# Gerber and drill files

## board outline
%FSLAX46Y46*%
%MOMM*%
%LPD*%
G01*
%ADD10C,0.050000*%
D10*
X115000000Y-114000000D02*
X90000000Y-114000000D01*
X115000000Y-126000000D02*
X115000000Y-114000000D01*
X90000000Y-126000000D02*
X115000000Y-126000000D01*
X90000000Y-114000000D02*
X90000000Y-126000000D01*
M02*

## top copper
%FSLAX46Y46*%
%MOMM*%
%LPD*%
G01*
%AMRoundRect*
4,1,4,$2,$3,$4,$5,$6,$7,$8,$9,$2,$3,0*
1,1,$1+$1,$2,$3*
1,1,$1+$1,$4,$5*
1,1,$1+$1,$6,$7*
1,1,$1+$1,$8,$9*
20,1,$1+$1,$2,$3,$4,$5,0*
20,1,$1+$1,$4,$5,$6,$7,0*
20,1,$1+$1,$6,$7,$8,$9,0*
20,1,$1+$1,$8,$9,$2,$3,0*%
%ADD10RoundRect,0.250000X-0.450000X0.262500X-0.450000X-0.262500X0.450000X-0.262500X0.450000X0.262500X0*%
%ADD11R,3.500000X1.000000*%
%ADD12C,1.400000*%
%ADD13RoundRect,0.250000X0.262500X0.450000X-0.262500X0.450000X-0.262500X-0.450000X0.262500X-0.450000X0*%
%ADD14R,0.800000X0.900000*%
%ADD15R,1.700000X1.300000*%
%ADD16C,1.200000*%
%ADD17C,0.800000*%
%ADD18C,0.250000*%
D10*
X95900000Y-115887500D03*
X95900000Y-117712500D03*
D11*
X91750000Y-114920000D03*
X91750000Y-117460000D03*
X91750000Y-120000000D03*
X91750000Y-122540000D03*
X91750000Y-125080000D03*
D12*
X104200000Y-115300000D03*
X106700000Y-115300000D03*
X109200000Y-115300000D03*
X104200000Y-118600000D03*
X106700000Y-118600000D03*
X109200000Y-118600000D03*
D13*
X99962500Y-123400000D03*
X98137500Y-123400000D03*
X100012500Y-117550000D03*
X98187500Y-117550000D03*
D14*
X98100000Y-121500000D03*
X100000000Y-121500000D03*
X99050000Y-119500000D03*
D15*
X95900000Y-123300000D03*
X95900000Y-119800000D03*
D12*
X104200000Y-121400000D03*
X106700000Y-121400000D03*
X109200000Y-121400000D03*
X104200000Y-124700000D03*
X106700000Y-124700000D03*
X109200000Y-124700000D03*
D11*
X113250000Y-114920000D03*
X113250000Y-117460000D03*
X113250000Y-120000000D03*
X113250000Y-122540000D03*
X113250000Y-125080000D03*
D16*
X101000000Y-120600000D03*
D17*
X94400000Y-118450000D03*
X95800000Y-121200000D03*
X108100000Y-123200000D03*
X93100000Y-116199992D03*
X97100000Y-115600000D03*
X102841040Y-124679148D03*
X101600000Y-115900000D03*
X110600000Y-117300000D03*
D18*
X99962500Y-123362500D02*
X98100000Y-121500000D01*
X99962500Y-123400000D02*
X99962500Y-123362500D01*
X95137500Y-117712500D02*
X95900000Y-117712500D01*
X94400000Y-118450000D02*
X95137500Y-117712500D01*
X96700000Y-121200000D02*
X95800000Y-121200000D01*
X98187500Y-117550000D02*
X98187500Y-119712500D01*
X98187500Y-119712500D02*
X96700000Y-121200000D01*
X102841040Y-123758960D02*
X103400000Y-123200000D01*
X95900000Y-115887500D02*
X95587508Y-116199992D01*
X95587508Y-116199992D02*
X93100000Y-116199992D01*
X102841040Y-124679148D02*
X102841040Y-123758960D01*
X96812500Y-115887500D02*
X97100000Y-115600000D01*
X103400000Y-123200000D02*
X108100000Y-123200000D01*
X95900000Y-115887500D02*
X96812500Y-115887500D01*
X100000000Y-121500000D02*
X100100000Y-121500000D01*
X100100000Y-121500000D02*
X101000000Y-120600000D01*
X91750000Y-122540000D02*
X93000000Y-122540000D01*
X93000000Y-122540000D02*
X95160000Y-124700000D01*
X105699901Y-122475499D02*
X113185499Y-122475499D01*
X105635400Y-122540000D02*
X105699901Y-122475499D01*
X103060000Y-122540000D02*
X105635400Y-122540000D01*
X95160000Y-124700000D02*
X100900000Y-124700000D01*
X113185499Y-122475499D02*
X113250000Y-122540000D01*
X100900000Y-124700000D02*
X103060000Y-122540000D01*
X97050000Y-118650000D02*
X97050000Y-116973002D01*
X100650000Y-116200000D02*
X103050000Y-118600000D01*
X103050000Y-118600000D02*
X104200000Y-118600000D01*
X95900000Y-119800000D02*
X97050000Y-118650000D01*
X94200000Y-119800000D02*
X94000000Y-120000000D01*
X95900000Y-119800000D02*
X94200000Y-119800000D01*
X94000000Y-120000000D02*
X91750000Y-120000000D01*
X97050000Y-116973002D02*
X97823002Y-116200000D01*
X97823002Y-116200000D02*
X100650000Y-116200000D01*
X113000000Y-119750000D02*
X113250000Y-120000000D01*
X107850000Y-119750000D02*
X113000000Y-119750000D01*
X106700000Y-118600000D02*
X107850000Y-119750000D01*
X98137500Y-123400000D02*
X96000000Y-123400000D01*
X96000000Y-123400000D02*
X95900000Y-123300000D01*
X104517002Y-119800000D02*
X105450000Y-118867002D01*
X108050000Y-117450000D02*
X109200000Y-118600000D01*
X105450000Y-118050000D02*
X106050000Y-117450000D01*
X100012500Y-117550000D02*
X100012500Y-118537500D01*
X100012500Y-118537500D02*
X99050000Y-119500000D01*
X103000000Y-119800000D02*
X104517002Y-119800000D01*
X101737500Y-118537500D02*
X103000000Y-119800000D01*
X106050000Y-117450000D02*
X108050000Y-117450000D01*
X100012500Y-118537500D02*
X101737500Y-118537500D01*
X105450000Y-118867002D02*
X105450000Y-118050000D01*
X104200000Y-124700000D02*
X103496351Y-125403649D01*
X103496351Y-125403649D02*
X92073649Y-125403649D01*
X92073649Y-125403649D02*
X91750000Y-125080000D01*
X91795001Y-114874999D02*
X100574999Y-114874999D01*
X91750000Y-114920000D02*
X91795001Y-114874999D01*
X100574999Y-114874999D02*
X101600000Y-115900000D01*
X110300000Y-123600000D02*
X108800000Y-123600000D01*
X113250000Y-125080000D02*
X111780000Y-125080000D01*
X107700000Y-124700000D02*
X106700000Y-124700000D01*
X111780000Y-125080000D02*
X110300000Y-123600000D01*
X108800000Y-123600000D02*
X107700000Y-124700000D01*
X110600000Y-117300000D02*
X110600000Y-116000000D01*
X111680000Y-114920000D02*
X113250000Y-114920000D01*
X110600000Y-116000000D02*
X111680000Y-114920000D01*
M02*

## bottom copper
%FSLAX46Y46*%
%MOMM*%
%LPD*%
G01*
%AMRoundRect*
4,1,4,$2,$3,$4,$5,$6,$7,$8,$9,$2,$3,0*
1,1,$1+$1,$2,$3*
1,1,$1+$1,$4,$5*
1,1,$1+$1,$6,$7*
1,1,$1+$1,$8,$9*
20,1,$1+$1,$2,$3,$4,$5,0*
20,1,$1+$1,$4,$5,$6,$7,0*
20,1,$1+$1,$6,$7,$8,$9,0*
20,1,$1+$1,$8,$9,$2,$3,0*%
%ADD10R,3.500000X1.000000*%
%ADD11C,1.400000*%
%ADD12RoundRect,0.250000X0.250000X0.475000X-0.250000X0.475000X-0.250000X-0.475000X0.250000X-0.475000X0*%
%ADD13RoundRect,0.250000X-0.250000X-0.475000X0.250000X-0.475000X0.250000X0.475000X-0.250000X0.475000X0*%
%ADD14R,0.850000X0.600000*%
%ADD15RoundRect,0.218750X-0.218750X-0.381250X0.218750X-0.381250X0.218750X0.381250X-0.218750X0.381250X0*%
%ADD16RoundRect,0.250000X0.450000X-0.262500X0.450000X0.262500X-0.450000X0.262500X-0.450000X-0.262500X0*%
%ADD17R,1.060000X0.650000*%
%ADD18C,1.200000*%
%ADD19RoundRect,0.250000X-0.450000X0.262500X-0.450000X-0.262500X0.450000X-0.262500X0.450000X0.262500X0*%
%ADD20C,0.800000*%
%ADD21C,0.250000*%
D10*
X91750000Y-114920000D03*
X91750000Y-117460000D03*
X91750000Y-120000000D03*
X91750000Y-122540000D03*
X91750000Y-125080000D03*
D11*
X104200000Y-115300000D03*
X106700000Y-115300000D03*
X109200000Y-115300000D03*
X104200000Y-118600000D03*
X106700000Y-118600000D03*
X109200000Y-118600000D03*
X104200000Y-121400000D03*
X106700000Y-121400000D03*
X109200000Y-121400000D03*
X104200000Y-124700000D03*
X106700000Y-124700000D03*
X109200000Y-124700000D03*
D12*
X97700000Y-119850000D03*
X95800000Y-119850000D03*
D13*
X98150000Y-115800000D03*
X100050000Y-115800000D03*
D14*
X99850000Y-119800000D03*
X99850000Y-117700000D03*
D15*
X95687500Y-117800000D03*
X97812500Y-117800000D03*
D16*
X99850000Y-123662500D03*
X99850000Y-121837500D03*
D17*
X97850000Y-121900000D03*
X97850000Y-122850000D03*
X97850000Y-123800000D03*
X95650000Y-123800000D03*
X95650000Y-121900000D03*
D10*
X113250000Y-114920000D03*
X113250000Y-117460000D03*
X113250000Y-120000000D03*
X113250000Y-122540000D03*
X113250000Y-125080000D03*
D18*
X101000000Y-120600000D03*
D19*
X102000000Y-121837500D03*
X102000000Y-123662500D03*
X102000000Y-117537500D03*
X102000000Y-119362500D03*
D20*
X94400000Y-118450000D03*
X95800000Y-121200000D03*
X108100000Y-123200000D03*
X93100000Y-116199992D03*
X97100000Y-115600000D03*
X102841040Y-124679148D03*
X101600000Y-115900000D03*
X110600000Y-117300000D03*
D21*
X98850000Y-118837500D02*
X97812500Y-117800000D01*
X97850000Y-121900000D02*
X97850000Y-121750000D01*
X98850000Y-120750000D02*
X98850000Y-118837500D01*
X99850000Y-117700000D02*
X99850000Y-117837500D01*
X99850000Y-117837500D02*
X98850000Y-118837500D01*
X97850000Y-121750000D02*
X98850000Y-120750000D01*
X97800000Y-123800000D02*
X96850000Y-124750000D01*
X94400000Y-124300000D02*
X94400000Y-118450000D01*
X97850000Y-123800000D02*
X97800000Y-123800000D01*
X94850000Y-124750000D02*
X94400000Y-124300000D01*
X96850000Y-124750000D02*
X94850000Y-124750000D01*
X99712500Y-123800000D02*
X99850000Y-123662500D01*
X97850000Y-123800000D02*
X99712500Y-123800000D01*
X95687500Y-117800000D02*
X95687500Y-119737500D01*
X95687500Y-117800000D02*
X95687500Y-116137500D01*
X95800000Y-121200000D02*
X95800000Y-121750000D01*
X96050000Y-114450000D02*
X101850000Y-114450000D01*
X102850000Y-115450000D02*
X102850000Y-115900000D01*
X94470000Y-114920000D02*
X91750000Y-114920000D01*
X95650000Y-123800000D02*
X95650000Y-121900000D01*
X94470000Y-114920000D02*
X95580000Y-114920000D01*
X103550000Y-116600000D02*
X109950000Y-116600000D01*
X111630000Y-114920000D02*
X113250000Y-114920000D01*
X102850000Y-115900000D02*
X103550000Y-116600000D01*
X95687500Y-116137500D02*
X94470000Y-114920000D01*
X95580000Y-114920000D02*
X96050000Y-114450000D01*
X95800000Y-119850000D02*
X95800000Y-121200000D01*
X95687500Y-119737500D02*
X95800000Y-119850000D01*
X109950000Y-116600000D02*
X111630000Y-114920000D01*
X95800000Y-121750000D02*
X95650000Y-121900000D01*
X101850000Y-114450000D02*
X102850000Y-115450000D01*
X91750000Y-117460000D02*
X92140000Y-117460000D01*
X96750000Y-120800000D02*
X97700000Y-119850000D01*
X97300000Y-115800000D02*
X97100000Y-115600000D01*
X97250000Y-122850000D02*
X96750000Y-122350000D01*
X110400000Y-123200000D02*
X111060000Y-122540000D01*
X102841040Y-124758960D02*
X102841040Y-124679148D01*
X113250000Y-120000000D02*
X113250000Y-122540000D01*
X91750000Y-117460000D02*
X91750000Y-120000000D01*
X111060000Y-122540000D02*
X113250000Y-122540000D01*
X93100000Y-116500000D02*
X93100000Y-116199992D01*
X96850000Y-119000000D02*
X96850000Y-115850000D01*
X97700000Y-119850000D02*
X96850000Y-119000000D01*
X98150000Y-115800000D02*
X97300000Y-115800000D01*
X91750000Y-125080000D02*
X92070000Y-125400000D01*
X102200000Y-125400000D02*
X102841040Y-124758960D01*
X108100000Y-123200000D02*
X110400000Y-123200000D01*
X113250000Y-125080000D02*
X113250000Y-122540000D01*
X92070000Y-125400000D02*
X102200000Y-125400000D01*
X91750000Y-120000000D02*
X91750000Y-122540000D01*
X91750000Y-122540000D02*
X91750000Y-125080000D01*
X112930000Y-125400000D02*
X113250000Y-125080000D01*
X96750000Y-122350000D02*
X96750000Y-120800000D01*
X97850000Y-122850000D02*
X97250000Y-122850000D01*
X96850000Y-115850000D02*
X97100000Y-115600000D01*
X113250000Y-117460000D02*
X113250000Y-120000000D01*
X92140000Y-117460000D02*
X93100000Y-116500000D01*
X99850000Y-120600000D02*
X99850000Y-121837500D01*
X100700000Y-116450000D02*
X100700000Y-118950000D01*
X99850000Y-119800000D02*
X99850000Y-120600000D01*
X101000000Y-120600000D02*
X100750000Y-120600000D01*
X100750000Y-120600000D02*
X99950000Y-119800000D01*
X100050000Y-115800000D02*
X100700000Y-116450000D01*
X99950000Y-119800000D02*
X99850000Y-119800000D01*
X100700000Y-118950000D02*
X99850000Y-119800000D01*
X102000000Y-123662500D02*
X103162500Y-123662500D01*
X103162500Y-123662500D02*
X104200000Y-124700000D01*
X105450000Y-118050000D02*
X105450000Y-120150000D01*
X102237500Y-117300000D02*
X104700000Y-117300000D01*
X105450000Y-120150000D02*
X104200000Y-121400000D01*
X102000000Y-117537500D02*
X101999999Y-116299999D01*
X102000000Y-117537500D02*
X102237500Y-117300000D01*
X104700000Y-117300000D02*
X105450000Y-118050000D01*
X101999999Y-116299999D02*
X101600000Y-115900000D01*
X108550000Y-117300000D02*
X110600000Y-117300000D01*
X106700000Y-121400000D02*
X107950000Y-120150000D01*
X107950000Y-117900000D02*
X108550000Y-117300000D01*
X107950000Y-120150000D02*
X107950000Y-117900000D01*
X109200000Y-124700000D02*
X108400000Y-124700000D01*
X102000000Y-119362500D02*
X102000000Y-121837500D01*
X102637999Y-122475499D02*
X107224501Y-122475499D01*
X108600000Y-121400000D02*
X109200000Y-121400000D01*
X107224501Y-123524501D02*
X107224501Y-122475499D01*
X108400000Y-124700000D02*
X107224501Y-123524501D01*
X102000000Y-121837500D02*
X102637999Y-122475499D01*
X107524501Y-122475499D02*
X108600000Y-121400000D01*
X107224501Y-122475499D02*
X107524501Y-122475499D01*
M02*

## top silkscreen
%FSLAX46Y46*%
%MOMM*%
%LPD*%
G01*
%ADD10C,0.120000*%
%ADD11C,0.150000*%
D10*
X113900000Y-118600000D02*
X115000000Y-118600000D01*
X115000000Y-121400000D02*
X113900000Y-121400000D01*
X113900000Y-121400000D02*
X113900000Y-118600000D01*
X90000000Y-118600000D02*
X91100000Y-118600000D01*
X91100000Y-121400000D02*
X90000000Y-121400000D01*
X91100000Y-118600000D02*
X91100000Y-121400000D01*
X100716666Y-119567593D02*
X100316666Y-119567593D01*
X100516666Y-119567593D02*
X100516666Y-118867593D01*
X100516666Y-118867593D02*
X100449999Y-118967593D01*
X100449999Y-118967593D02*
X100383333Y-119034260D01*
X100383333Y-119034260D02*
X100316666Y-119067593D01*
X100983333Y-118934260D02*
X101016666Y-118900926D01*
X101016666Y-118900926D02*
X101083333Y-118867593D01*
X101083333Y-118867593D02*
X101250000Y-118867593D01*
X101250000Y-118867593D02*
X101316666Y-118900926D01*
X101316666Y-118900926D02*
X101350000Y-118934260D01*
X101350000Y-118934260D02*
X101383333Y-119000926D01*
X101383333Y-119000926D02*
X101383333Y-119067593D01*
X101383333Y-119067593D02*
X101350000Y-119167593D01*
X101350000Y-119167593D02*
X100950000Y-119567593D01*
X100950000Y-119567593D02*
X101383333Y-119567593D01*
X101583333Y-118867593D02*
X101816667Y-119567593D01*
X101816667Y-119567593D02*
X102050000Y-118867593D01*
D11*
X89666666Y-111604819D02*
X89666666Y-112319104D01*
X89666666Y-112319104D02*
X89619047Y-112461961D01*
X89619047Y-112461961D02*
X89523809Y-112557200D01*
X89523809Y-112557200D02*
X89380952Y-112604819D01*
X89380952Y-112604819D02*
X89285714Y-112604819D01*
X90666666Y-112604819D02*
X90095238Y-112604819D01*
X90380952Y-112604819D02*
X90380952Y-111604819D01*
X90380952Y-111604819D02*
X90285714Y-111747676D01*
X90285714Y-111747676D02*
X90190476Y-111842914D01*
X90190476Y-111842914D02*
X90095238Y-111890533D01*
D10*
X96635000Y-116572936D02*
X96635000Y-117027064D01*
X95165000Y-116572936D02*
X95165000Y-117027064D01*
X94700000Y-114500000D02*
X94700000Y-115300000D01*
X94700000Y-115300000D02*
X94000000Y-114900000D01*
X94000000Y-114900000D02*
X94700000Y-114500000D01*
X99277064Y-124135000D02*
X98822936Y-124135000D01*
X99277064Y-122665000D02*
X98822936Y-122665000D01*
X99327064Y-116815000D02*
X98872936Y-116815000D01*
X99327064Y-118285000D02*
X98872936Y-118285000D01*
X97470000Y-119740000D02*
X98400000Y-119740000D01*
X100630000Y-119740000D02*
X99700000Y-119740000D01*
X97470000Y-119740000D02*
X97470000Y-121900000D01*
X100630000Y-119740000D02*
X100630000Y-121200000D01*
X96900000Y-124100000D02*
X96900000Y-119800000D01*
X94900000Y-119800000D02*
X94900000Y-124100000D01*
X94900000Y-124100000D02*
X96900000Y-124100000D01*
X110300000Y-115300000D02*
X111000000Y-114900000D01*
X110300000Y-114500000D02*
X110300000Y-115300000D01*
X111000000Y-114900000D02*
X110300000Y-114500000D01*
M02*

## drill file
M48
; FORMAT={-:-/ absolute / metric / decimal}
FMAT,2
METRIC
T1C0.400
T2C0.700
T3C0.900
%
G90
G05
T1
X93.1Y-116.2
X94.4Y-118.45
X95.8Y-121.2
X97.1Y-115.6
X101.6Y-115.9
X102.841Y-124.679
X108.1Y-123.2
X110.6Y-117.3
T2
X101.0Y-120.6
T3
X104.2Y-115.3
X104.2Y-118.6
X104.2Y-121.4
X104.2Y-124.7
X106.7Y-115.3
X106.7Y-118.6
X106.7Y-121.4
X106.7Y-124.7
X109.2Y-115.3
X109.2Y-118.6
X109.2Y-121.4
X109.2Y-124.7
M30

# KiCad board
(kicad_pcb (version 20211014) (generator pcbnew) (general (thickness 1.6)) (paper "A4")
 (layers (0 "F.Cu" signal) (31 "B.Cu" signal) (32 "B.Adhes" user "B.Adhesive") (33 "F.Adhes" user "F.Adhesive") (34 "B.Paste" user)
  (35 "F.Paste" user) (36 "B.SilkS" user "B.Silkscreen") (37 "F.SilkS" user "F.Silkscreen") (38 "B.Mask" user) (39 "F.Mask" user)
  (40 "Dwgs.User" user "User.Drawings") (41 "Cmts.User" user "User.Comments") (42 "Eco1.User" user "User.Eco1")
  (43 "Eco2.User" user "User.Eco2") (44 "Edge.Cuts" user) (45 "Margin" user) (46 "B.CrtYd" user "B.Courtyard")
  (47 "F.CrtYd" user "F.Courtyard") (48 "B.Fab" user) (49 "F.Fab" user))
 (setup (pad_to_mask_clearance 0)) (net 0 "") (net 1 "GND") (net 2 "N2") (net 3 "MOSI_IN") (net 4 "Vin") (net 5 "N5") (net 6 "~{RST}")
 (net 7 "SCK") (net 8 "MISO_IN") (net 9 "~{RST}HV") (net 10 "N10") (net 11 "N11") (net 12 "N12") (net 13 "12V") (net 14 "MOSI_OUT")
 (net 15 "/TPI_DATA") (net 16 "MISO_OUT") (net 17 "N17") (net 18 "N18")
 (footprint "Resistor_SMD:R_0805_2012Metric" (layer "F.Cu") (at 95.9 116.8 -90)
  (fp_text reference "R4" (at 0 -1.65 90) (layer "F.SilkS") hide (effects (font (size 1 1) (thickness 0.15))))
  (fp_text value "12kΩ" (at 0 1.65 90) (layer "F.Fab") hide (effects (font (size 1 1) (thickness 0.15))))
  (fp_line (start -0.227064 -0.735) (end 0.227064 -0.735) (layer "F.SilkS") (width 0.12))
  (fp_line (start -0.227064 0.735) (end 0.227064 0.735) (layer "F.SilkS") (width 0.12))
  (pad "1" smd roundrect locked (at -0.9125 0 270) (size 1.025 1.4) (layers "F.Cu" "F.Paste" "F.Mask") (roundrect_rratio 0.243902)
   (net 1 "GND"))
  (pad "2" smd roundrect locked (at 0.9125 0 270) (size 1.025 1.4) (layers "F.Cu" "F.Paste" "F.Mask") (roundrect_rratio 0.243902)
   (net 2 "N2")))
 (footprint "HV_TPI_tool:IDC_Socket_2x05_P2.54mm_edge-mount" (layer "F.Cu") (at 90 120)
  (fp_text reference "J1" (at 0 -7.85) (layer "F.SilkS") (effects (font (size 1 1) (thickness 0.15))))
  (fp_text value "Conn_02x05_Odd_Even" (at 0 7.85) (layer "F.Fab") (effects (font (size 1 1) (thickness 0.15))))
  (fp_line (start 4.7 -5.5) (end 4.7 -4.7) (layer "F.SilkS") (width 0.12))
  (fp_line (start 4.7 -4.7) (end 4 -5.1) (layer "F.SilkS") (width 0.12))
  (fp_line (start 4 -5.1) (end 4.7 -5.5) (layer "F.SilkS") (width 0.12))
  (pad "1" smd rect (at 1.75 -5.08) (size 3.5 1) (layers "F.Cu" "F.Paste" "F.Mask") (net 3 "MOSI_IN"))
  (pad "2" smd rect (at 1.75 -5.08) (size 3.5 1) (layers "B.Cu" "B.Paste" "B.Mask") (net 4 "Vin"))
  (pad "3" smd rect (at 1.75 -2.54) (size 3.5 1) (layers "F.Cu" "F.Paste" "F.Mask") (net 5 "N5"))
  (pad "4" smd rect (at 1.75 -2.54) (size 3.5 1) (layers "B.Cu" "B.Paste" "B.Mask") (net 1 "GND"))
  (pad "5" smd rect (at 1.75 0) (size 3.5 1) (layers "F.Cu" "F.Paste" "F.Mask") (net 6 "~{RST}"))
  (pad "6" smd rect (at 1.75 0) (size 3.5 1) (layers "B.Cu" "B.Paste" "B.Mask") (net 1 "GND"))
  (pad "7" smd rect (at 1.75 2.54) (size 3.5 1) (layers "F.Cu" "F.Paste" "F.Mask") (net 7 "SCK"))
  (pad "8" smd rect (at 1.75 2.54) (size 3.5 1) (layers "B.Cu" "B.Paste" "B.Mask") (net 1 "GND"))
  (pad "9" smd rect (at 1.75 5.08) (size 3.5 1) (layers "F.Cu" "F.Paste" "F.Mask") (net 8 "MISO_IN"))
  (pad "10" smd rect (at 1.75 5.08) (size 3.5 1) (layers "B.Cu" "B.Paste" "B.Mask") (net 1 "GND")))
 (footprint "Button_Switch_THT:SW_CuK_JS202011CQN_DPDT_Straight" (layer "F.Cu") (at 104.2 115.3)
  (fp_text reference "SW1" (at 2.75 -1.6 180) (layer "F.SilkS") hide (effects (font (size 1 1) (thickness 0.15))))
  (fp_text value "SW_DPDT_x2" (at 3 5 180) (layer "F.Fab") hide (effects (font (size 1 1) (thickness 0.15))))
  (pad "1" thru_hole circle locked (at 0 0) (size 1.4 1.4) (drill 0.9) (layers *.Cu *.Mask))
  (pad "2" thru_hole circle locked (at 2.5 0) (size 1.4 1.4) (drill 0.9) (layers *.Cu *.Mask))
  (pad "3" thru_hole circle locked (at 5 0) (size 1.4 1.4) (drill 0.9) (layers *.Cu *.Mask))
  (pad "4" thru_hole circle locked (at 0 3.3) (size 1.4 1.4) (drill 0.9) (layers *.Cu *.Mask) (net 6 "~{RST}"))
  (pad "5" thru_hole circle locked (at 2.5 3.3) (size 1.4 1.4) (drill 0.9) (layers *.Cu *.Mask) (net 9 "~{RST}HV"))
  (pad "6" thru_hole circle locked (at 5 3.3) (size 1.4 1.4) (drill 0.9) (layers *.Cu *.Mask) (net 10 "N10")))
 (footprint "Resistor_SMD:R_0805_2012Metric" (layer "F.Cu") (at 99.05 123.4 180)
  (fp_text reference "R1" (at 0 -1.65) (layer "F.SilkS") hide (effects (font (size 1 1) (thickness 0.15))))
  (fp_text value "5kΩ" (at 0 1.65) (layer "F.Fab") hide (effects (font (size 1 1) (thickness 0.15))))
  (fp_line (start -0.227064 -0.735) (end 0.227064 -0.735) (layer "F.SilkS") (width 0.12))
  (fp_line (start -0.227064 0.735) (end 0.227064 0.735) (layer "F.SilkS") (width 0.12))
  (pad "1" smd roundrect locked (at -0.9125 0 180) (size 1.025 1.4) (layers "F.Cu" "F.Paste" "F.Mask") (roundrect_rratio 0.243902)
   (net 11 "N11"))
  (pad "2" smd roundrect locked (at 0.9125 0 180) (size 1.025 1.4) (layers "F.Cu" "F.Paste" "F.Mask") (roundrect_rratio 0.243902)
   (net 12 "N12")))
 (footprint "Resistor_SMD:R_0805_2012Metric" (layer "F.Cu") (at 99.1 117.55 180)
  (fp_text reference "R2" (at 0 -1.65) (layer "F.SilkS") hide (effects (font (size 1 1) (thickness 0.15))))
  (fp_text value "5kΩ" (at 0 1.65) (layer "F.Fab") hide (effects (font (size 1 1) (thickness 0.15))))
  (fp_line (start -0.227064 0.735) (end 0.227064 0.735) (layer "F.SilkS") (width 0.12))
  (fp_line (start -0.227064 -0.735) (end 0.227064 -0.735) (layer "F.SilkS") (width 0.12))
  (pad "1" smd roundrect locked (at -0.9125 0 180) (size 1.025 1.4) (layers "F.Cu" "F.Paste" "F.Mask") (roundrect_rratio 0.243902)
   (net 10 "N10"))
  (pad "2" smd roundrect locked (at 0.9125 0 180) (size 1.025 1.4) (layers "F.Cu" "F.Paste" "F.Mask") (roundrect_rratio 0.243902)
   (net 4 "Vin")))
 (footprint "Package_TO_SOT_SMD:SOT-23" (layer "F.Cu") (at 99.05 120.5 90)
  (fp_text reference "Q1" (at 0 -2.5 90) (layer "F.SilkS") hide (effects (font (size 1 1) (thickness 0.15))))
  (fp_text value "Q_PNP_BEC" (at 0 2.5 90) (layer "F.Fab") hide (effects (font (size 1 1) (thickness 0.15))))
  (fp_line (start 0.76 -1.58) (end 0.76 -0.65) (layer "F.SilkS") (width 0.12))
  (fp_line (start 0.76 1.58) (end 0.76 0.65) (layer "F.SilkS") (width 0.12))
  (fp_line (start 0.76 -1.58) (end -1.4 -1.58) (layer "F.SilkS") (width 0.12))
  (fp_line (start 0.76 1.58) (end -0.7 1.58) (layer "F.SilkS") (width 0.12))
  (pad "1" smd rect locked (at -1 -0.95 90) (size 0.9 0.8) (layers "F.Cu" "F.Paste" "F.Mask") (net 11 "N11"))
  (pad "2" smd rect locked (at -1 0.95 90) (size 0.9 0.8) (layers "F.Cu" "F.Paste" "F.Mask") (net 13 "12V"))
  (pad "3" smd rect locked (at 1 0 90) (size 0.9 0.8) (layers "F.Cu" "F.Paste" "F.Mask") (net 10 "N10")))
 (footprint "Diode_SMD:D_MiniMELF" (layer "F.Cu") (at 95.9 121.55 90)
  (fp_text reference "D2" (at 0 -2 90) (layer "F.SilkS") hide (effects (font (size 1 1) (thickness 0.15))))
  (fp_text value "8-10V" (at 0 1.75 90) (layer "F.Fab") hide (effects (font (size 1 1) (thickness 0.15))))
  (fp_line (start -2.55 1) (end 1.75 1) (layer "F.SilkS") (width 0.12))
  (fp_line (start 1.75 -1) (end -2.55 -1) (layer "F.SilkS") (width 0.12))
  (fp_line (start -2.55 -1) (end -2.55 1) (layer "F.SilkS") (width 0.12))
  (pad "1" smd rect locked (at -1.75 0 90) (size 1.3 1.7) (layers "F.Cu" "F.Paste" "F.Mask") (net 12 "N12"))
  (pad "2" smd rect locked (at 1.75 0 90) (size 1.3 1.7) (layers "F.Cu" "F.Paste" "F.Mask") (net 6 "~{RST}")))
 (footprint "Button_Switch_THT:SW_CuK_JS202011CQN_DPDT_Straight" (layer "F.Cu") (at 104.2 121.4)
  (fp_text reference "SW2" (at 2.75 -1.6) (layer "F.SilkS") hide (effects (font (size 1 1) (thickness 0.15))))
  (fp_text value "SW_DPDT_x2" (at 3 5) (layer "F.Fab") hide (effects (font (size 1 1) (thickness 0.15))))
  (pad "1" thru_hole circle (at 0 0) (size 1.4 1.4) (drill 0.9) (layers *.Cu *.Mask) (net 3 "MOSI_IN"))
  (pad "2" thru_hole circle (at 2.5 0) (size 1.4 1.4) (drill 0.9) (layers *.Cu *.Mask) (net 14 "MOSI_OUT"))
  (pad "3" thru_hole circle (at 5 0) (size 1.4 1.4) (drill 0.9) (layers *.Cu *.Mask) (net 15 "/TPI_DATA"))
  (pad "4" thru_hole circle (at 0 3.3) (size 1.4 1.4) (drill 0.9) (layers *.Cu *.Mask) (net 8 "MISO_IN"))
  (pad "5" thru_hole circle (at 2.5 3.3) (size 1.4 1.4) (drill 0.9) (layers *.Cu *.Mask) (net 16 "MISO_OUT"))
  (pad "6" thru_hole circle (at 5 3.3) (size 1.4 1.4) (drill 0.9) (layers *.Cu *.Mask) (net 15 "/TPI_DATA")))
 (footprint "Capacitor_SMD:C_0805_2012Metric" (layer "B.Cu") (at 96.75 119.85 180)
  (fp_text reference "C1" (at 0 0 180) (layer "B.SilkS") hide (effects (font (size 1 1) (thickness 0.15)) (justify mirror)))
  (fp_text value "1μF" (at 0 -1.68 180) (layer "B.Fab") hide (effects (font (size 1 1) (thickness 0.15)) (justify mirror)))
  (pad "1" smd roundrect locked (at -0.95 0 180) (size 1 1.45) (layers "B.Cu" "B.Paste" "B.Mask") (roundrect_rratio 0.25) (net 1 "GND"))
  (pad "2" smd roundrect locked (at 0.95 0 180) (size 1 1.45) (layers "B.Cu" "B.Paste" "B.Mask") (roundrect_rratio 0.25) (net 4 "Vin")))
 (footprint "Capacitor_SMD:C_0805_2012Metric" (layer "B.Cu") (at 99.1 115.8)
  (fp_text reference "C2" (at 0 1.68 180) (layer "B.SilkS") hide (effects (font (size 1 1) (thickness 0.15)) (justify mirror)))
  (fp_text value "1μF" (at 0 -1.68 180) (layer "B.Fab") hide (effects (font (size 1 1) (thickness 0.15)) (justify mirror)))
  (pad "1" smd roundrect locked (at -0.95 0) (size 1 1.45) (layers "B.Cu" "B.Paste" "B.Mask") (roundrect_rratio 0.25) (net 1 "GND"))
  (pad "2" smd roundrect locked (at 0.95 0) (size 1 1.45) (layers "B.Cu" "B.Paste" "B.Mask") (roundrect_rratio 0.25) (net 13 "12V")))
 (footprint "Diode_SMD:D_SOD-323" (layer "B.Cu") (at 99.85 118.75 90)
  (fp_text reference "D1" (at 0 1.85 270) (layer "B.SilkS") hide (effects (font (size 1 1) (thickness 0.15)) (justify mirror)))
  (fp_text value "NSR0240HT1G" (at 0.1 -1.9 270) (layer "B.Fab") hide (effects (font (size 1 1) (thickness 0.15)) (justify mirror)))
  (pad "1" smd rect locked (at -1.05 0 90) (size 0.6 0.85) (layers "B.Cu" "B.Paste" "B.Mask") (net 13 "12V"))
  (pad "2" smd rect locked (at 1.05 0 90) (size 0.6 0.85) (layers "B.Cu" "B.Paste" "B.Mask") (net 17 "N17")))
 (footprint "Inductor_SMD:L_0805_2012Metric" (layer "B.Cu") (at 96.75 117.8)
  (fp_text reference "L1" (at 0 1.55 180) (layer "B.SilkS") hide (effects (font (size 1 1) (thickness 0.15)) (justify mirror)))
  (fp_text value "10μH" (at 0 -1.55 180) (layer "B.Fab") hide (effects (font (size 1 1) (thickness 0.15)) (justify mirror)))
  (pad "1" smd roundrect locked (at -1.0625 0) (size 0.875 1.2) (layers "B.Cu" "B.Paste" "B.Mask") (roundrect_rratio 0.25) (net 4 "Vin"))
  (pad "2" smd roundrect locked (at 1.0625 0) (size 0.875 1.2) (layers "B.Cu" "B.Paste" "B.Mask") (roundrect_rratio 0.25) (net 17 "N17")))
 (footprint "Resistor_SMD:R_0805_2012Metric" (layer "B.Cu") (at 99.85 122.75 90)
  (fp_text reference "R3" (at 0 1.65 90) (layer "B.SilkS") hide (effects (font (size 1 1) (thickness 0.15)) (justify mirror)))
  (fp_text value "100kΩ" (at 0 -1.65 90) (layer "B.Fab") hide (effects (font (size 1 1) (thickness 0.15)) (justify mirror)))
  (pad "1" smd roundrect locked (at -0.9125 0 90) (size 1.025 1.4) (layers "B.Cu" "B.Paste" "B.Mask") (roundrect_rratio 0.243902)
   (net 2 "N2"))
  (pad "2" smd roundrect locked (at 0.9125 0 90) (size 1.025 1.4) (layers "B.Cu" "B.Paste" "B.Mask") (roundrect_rratio 0.243902)
   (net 13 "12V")))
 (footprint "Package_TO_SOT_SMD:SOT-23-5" (layer "B.Cu") (at 96.75 122.85 180)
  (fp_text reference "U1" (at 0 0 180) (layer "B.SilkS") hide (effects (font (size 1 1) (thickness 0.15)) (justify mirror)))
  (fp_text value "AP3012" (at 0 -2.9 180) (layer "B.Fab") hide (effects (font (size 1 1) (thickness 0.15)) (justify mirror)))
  (pad "1" smd rect locked (at -1.1 0.95 180) (size 1.06 0.65) (layers "B.Cu" "B.Paste" "B.Mask") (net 17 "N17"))
  (pad "2" smd rect locked (at -1.1 0 180) (size 1.06 0.65) (layers "B.Cu" "B.Paste" "B.Mask") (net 1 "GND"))
  (pad "3" smd rect locked (at -1.1 -0.95 180) (size 1.06 0.65) (layers "B.Cu" "B.Paste" "B.Mask") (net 2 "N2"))
  (pad "4" smd rect locked (at 1.1 -0.95 180) (size 1.06 0.65) (layers "B.Cu" "B.Paste" "B.Mask") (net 4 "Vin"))
  (pad "5" smd rect locked (at 1.1 0.95 180) (size 1.06 0.65) (layers "B.Cu" "B.Paste" "B.Mask") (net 4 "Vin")))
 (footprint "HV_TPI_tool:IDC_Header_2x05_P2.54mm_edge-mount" (layer "B.Cu") (at 115 120 180)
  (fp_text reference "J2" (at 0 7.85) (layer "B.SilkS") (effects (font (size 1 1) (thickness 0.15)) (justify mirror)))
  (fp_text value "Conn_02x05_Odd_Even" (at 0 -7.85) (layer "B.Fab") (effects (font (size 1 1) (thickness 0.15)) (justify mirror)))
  (fp_line (start 4.7 4.7) (end 4 5.1) (layer "F.SilkS") (width 0.12))
  (fp_line (start 4.7 5.5) (end 4.7 4.7) (layer "F.SilkS") (width 0.12))
  (fp_line (start 4 5.1) (end 4.7 5.5) (layer "F.SilkS") (width 0.12))
  (pad "1" smd rect (at 1.75 5.08 180) (size 3.5 1) (layers "F.Cu" "F.Paste" "F.Mask") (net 14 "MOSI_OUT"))
  (pad "2" smd rect (at 1.75 5.08 180) (size 3.5 1) (layers "B.Cu" "B.Paste" "B.Mask") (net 4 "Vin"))
  (pad "3" smd rect (at 1.75 2.54 180) (size 3.5 1) (layers "F.Cu" "F.Paste" "F.Mask") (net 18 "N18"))
  (pad "4" smd rect (at 1.75 2.54 180) (size 3.5 1) (layers "B.Cu" "B.Paste" "B.Mask") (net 1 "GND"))
  (pad "5" smd rect (at 1.75 0 180) (size 3.5 1) (layers "F.Cu" "F.Paste" "F.Mask") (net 9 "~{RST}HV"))
  (pad "6" smd rect (at 1.75 0 180) (size 3.5 1) (layers "B.Cu" "B.Paste" "B.Mask") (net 1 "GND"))
  (pad "7" smd rect (at 1.75 -2.54 180) (size 3.5 1) (layers "F.Cu" "F.Paste" "F.Mask") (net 7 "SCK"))
  (pad "8" smd rect (at 1.75 -2.54 180) (size 3.5 1) (layers "B.Cu" "B.Paste" "B.Mask") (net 1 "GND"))
  (pad "9" smd rect (at 1.75 -5.08 180) (size 3.5 1) (layers "F.Cu" "F.Paste" "F.Mask") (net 16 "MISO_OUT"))
  (pad "10" smd rect (at 1.75 -5.08 180) (size 3.5 1) (layers "B.Cu" "B.Paste" "B.Mask") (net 1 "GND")))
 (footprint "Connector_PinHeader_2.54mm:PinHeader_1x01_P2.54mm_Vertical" (layer "B.Cu") (at 101 120.6)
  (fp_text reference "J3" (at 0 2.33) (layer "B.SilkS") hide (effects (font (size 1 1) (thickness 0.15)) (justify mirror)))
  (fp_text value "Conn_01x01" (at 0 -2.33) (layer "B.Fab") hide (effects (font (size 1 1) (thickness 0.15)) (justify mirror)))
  (pad "1" thru_hole circle locked (at 0 0) (size 1.2 1.2) (drill 0.7) (layers *.Cu *.Mask) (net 13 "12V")))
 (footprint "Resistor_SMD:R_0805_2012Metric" (layer "B.Cu") (at 102 122.75 -90)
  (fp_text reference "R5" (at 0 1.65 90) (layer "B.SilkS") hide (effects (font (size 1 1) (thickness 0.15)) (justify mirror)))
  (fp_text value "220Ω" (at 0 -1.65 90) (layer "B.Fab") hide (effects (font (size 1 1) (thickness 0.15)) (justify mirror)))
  (pad "1" smd roundrect locked (at -0.9125 0 270) (size 1.025 1.4) (layers "B.Cu" "B.Paste" "B.Mask") (roundrect_rratio 0.243902)
   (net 15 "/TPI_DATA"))
  (pad "2" smd roundrect locked (at 0.9125 0 270) (size 1.025 1.4) (layers "B.Cu" "B.Paste" "B.Mask") (roundrect_rratio 0.243902)
   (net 8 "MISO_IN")))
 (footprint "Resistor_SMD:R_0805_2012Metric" (layer "B.Cu") (at 102 118.45 -90)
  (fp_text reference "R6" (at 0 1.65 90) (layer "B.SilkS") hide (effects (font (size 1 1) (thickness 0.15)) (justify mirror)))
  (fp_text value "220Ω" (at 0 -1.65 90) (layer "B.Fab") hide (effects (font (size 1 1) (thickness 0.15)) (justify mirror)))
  (pad "1" smd roundrect locked (at -0.9125 0 270) (size 1.025 1.4) (layers "B.Cu" "B.Paste" "B.Mask") (roundrect_rratio 0.243902)
   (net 3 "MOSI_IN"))
  (pad "2" smd roundrect locked (at 0.9125 0 270) (size 1.025 1.4) (layers "B.Cu" "B.Paste" "B.Mask") (roundrect_rratio 0.243902)
   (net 15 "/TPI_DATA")))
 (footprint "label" (layer "B.Cu") (at 94.35 119.95 -90)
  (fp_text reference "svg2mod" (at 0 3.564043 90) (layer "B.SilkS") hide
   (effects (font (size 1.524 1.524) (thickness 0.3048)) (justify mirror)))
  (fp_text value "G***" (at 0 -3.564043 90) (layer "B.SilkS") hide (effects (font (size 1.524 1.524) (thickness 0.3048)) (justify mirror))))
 (gr_line (start 113.9 118.6) (end 115 118.6) (layer "F.SilkS") (width 0.12))
 (gr_line (start 115 121.4) (end 113.9 121.4) (layer "F.SilkS") (width 0.12))
 (gr_line (start 113.9 121.4) (end 113.9 118.6) (layer "F.SilkS") (width 0.12))
 (gr_line (start 90 118.6) (end 91.1 118.6) (layer "F.SilkS") (width 0.12))
 (gr_line (start 91.1 121.4) (end 90 121.4) (layer "F.SilkS") (width 0.12))
 (gr_line (start 91.1 118.6) (end 91.1 121.4) (layer "F.SilkS") (width 0.12))
 (gr_line (start 115 114) (end 90 114) (layer "Edge.Cuts") (width 0.05))
 (gr_line (start 115 126) (end 115 114) (layer "Edge.Cuts") (width 0.05))
 (gr_line (start 90 126) (end 115 126) (layer "Edge.Cuts") (width 0.05))
 (gr_line (start 90 114) (end 90 126) (layer "Edge.Cuts") (width 0.05))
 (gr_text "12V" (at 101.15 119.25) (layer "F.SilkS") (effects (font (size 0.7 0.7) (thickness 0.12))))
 (segment (start 99.9625 123.3625) (end 98.1 121.5) (width 0.25) (layer "F.Cu") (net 11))
 (segment (start 99.9625 123.4) (end 99.9625 123.3625) (width 0.25) (layer "F.Cu") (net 11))
 (segment (start 98.85 118.8375) (end 97.8125 117.8) (width 0.25) (layer "B.Cu") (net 17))
 (segment (start 97.85 121.9) (end 97.85 121.75) (width 0.25) (layer "B.Cu") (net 17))
 (segment (start 98.85 120.75) (end 98.85 118.8375) (width 0.25) (layer "B.Cu") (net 17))
 (segment (start 99.85 117.7) (end 99.85 117.8375) (width 0.25) (layer "B.Cu") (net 17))
 (segment (start 99.85 117.8375) (end 98.85 118.8375) (width 0.25) (layer "B.Cu") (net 17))
 (segment (start 97.85 121.75) (end 98.85 120.75) (width 0.25) (layer "B.Cu") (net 17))
 (segment (start 95.1375 117.7125) (end 95.9 117.7125) (width 0.25) (layer "F.Cu") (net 2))
 (segment (start 94.4 118.45) (end 95.1375 117.7125) (width 0.25) (layer "F.Cu") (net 2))
 (via (at 94.4 118.45) (size 0.8) (drill 0.4) (layers "F.Cu" "B.Cu") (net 2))
 (segment (start 97.8 123.8) (end 96.85 124.75) (width 0.25) (layer "B.Cu") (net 2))
 (segment (start 94.4 124.3) (end 94.4 118.45) (width 0.25) (layer "B.Cu") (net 2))
 (segment (start 97.85 123.8) (end 97.8 123.8) (width 0.25) (layer "B.Cu") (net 2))
 (segment (start 94.85 124.75) (end 94.4 124.3) (width 0.25) (layer "B.Cu") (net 2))
 (segment (start 96.85 124.75) (end 94.85 124.75) (width 0.25) (layer "B.Cu") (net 2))
 (segment (start 99.7125 123.8) (end 99.85 123.6625) (width 0.25) (layer "B.Cu") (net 2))
 (segment (start 97.85 123.8) (end 99.7125 123.8) (width 0.25) (layer "B.Cu") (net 2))
 (segment (start 96.7 121.2) (end 95.8 121.2) (width 0.25) (layer "F.Cu") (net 4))
 (segment (start 98.1875 117.55) (end 98.1875 119.7125) (width 0.25) (layer "F.Cu") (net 4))
 (segment (start 98.1875 119.7125) (end 96.7 121.2) (width 0.25) (layer "F.Cu") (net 4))
 (via (at 95.8 121.2) (size 0.8) (drill 0.4) (layers "F.Cu" "B.Cu") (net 4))
 (segment (start 95.6875 117.8) (end 95.6875 119.7375) (width 0.25) (layer "B.Cu") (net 4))
 (segment (start 95.6875 117.8) (end 95.6875 116.1375) (width 0.25) (layer "B.Cu") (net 4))
 (segment (start 95.8 121.2) (end 95.8 121.75) (width 0.25) (layer "B.Cu") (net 4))
 (segment (start 96.05 114.45) (end 101.85 114.45) (width 0.25) (layer "B.Cu") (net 4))
 (segment (start 102.85 115.45) (end 102.85 115.9) (width 0.25) (layer "B.Cu") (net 4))
 (segment (start 94.47 114.92) (end 91.75 114.92) (width 0.25) (layer "B.Cu") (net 4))
 (segment (start 95.65 123.8) (end 95.65 121.9) (width 0.25) (layer "B.Cu") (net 4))
 (segment (start 94.47 114.92) (end 95.58 114.92) (width 0.25) (layer "B.Cu") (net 4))
 (segment (start 103.55 116.6) (end 109.95 116.6) (width 0.25) (layer "B.Cu") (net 4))
 (segment (start 111.63 114.92) (end 113.25 114.92) (width 0.25) (layer "B.Cu") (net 4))
 (segment (start 102.85 115.9) (end 103.55 116.6) (width 0.25) (layer "B.Cu") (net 4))
 (segment (start 95.6875 116.1375) (end 94.47 114.92) (width 0.25) (layer "B.Cu") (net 4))
 (segment (start 95.58 114.92) (end 96.05 114.45) (width 0.25) (layer "B.Cu") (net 4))
 (segment (start 95.8 119.85) (end 95.8 121.2) (width 0.25) (layer "B.Cu") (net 4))
 (segment (start 95.6875 119.7375) (end 95.8 119.85) (width 0.25) (layer "B.Cu") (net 4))
 (segment (start 109.95 116.6) (end 111.63 114.92) (width 0.25) (layer "B.Cu") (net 4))
 (segment (start 95.8 121.75) (end 95.65 121.9) (width 0.25) (layer "B.Cu") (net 4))
 (segment (start 101.85 114.45) (end 102.85 115.45) (width 0.25) (layer "B.Cu") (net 4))
 (segment (start 102.84104 123.75896) (end 103.4 123.2) (width 0.25) (layer "F.Cu") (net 1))
 (segment (start 95.9 115.8875) (end 95.587508 116.199992) (width 0.25) (layer "F.Cu") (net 1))
 (segment (start 95.587508 116.199992) (end 93.1 116.199992) (width 0.25) (layer "F.Cu") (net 1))
 (segment (start 102.84104 124.679148) (end 102.84104 123.75896) (width 0.25) (layer "F.Cu") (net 1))
 (segment (start 96.8125 115.8875) (end 97.1 115.6) (width 0.25) (layer "F.Cu") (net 1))
 (segment (start 103.4 123.2) (end 108.1 123.2) (width 0.25) (layer "F.Cu") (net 1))
 (segment (start 95.9 115.8875) (end 96.8125 115.8875) (width 0.25) (layer "F.Cu") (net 1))
 (via (at 108.1 123.2) (size 0.8) (drill 0.4) (layers "F.Cu" "B.Cu") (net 1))
 (via (at 93.1 116.199992) (size 0.8) (drill 0.4) (layers "F.Cu" "B.Cu") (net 1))
 (via (at 97.1 115.6) (size 0.8) (drill 0.4) (layers "F.Cu" "B.Cu") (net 1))
 (via (at 102.84104 124.679148) (size 0.8) (drill 0.4) (layers "F.Cu" "B.Cu") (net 1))
 (segment (start 91.75 117.46) (end 92.14 117.46) (width 0.25) (layer "B.Cu") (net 1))
 (segment (start 96.75 120.8) (end 97.7 119.85) (width 0.25) (layer "B.Cu") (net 1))
 (segment (start 97.3 115.8) (end 97.1 115.6) (width 0.25) (layer "B.Cu") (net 1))
 (segment (start 97.25 122.85) (end 96.75 122.35) (width 0.25) (layer "B.Cu") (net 1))
 (segment (start 110.4 123.2) (end 111.06 122.54) (width 0.25) (layer "B.Cu") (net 1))
 (segment (start 102.84104 124.75896) (end 102.84104 124.679148) (width 0.25) (layer "B.Cu") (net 1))
 (segment (start 113.25 120) (end 113.25 122.54) (width 0.25) (layer "B.Cu") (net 1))
 (segment (start 91.75 117.46) (end 91.75 120) (width 0.25) (layer "B.Cu") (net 1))
 (segment (start 111.06 122.54) (end 113.25 122.54) (width 0.25) (layer "B.Cu") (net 1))
 (segment (start 93.1 116.5) (end 93.1 116.199992) (width 0.25) (layer "B.Cu") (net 1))
 (segment (start 96.85 119) (end 96.85 115.85) (width 0.25) (layer "B.Cu") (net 1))
 (segment (start 97.7 119.85) (end 96.85 119) (width 0.25) (layer "B.Cu") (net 1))
 (segment (start 98.15 115.8) (end 97.3 115.8) (width 0.25) (layer "B.Cu") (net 1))
 (segment (start 91.75 125.08) (end 92.07 125.4) (width 0.25) (layer "B.Cu") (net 1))
 (segment (start 102.2 125.4) (end 102.84104 124.75896) (width 0.25) (layer "B.Cu") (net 1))
 (segment (start 108.1 123.2) (end 110.4 123.2) (width 0.25) (layer "B.Cu") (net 1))
 (segment (start 113.25 125.08) (end 113.25 122.54) (width 0.25) (layer "B.Cu") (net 1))
 (segment (start 92.07 125.4) (end 102.2 125.4) (width 0.25) (layer "B.Cu") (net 1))
 (segment (start 91.75 120) (end 91.75 122.54) (width 0.25) (layer "B.Cu") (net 1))
 (segment (start 91.75 122.54) (end 91.75 125.08) (width 0.25) (layer "B.Cu") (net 1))
 (segment (start 112.93 125.4) (end 113.25 125.08) (width 0.25) (layer "B.Cu") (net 1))
 (segment (start 96.75 122.35) (end 96.75 120.8) (width 0.25) (layer "B.Cu") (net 1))
 (segment (start 97.85 122.85) (end 97.25 122.85) (width 0.25) (layer "B.Cu") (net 1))
 (segment (start 96.85 115.85) (end 97.1 115.6) (width 0.25) (layer "B.Cu") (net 1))
 (segment (start 113.25 117.46) (end 113.25 120) (width 0.25) (layer "B.Cu") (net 1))
 (segment (start 92.14 117.46) (end 93.1 116.5) (width 0.25) (layer "B.Cu") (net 1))
 (segment (start 100 121.5) (end 100.1 121.5) (width 0.25) (layer "F.Cu") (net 13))
 (segment (start 100.1 121.5) (end 101 120.6) (width 0.25) (layer "F.Cu") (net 13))
 (segment (start 99.85 120.6) (end 99.85 121.8375) (width 0.25) (layer "B.Cu") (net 13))
 (segment (start 100.7 116.45) (end 100.7 118.95) (width 0.25) (layer "B.Cu") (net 13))
 (segment (start 99.85 119.8) (end 99.85 120.6) (width 0.25) (layer "B.Cu") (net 13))
 (segment (start 101 120.6) (end 100.75 120.6) (width 0.25) (layer "B.Cu") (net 13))
 (segment (start 100.75 120.6) (end 99.95 119.8) (width 0.25) (layer "B.Cu") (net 13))
 (segment (start 100.05 115.8) (end 100.7 116.45) (width 0.25) (layer "B.Cu") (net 13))
 (segment (start 99.95 119.8) (end 99.85 119.8) (width 0.25) (layer "B.Cu") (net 13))
 (segment (start 100.7 118.95) (end 99.85 119.8) (width 0.25) (layer "B.Cu") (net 13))
 (segment (start 91.75 122.54) (end 93 122.54) (width 0.25) (layer "F.Cu") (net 7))
 (segment (start 93 122.54) (end 95.16 124.7) (width 0.25) (layer "F.Cu") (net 7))
 (segment (start 105.699901 122.475499) (end 113.185499 122.475499) (width 0.25) (layer "F.Cu") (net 7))
 (segment (start 105.6354 122.54) (end 105.699901 122.475499) (width 0.25) (layer "F.Cu") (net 7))
 (segment (start 103.06 122.54) (end 105.6354 122.54) (width 0.25) (layer "F.Cu") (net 7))
 (segment (start 95.16 124.7) (end 100.9 124.7) (width 0.25) (layer "F.Cu") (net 7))
 (segment (start 113.185499 122.475499) (end 113.25 122.54) (width 0.25) (layer "F.Cu") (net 7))
 (segment (start 100.9 124.7) (end 103.06 122.54) (width 0.25) (layer "F.Cu") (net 7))
 (segment (start 97.05 118.65) (end 97.05 116.973002) (width 0.25) (layer "F.Cu") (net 6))
 (segment (start 100.65 116.2) (end 103.05 118.6) (width 0.25) (layer "F.Cu") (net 6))
 (segment (start 103.05 118.6) (end 104.2 118.6) (width 0.25) (layer "F.Cu") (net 6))
 (segment (start 95.9 119.8) (end 97.05 118.65) (width 0.25) (layer "F.Cu") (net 6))
 (segment (start 94.2 119.8) (end 94 120) (width 0.25) (layer "F.Cu") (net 6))
 (segment (start 95.9 119.8) (end 94.2 119.8) (width 0.25) (layer "F.Cu") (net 6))
 (segment (start 94 120) (end 91.75 120) (width 0.25) (layer "F.Cu") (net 6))
 (segment (start 97.05 116.973002) (end 97.823002 116.2) (width 0.25) (layer "F.Cu") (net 6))
 (segment (start 97.823002 116.2) (end 100.65 116.2) (width 0.25) (layer "F.Cu") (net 6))
 (segment (start 113 119.75) (end 113.25 120) (width 0.25) (layer "F.Cu") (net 9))
 (segment (start 107.85 119.75) (end 113 119.75) (width 0.25) (layer "F.Cu") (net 9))
 (segment (start 106.7 118.6) (end 107.85 119.75) (width 0.25) (layer "F.Cu") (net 9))
 (segment (start 98.1375 123.4) (end 96 123.4) (width 0.25) (layer "F.Cu") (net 12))
 (segment (start 96 123.4) (end 95.9 123.3) (width 0.25) (layer "F.Cu") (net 12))
 (segment (start 104.517002 119.8) (end 105.45 118.867002) (width 0.25) (layer "F.Cu") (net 10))
 (segment (start 108.05 117.45) (end 109.2 118.6) (width 0.25) (layer "F.Cu") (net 10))
 (segment (start 105.45 118.05) (end 106.05 117.45) (width 0.25) (layer "F.Cu") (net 10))
 (segment (start 100.0125 117.55) (end 100.0125 118.5375) (width 0.25) (layer "F.Cu") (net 10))
 (segment (start 100.0125 118.5375) (end 99.05 119.5) (width 0.25) (layer "F.Cu") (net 10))
 (segment (start 103 119.8) (end 104.517002 119.8) (width 0.25) (layer "F.Cu") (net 10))
 (segment (start 101.7375 118.5375) (end 103 119.8) (width 0.25) (layer "F.Cu") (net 10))
 (segment (start 106.05 117.45) (end 108.05 117.45) (width 0.25) (layer "F.Cu") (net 10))
 (segment (start 100.0125 118.5375) (end 101.7375 118.5375) (width 0.25) (layer "F.Cu") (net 10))
 (segment (start 105.45 118.867002) (end 105.45 118.05) (width 0.25) (layer "F.Cu") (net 10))
 (segment (start 104.2 124.7) (end 103.496351 125.403649) (width 0.25) (layer "F.Cu") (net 8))
 (segment (start 103.496351 125.403649) (end 92.073649 125.403649) (width 0.25) (layer "F.Cu") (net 8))
 (segment (start 92.073649 125.403649) (end 91.75 125.08) (width 0.25) (layer "F.Cu") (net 8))
 (segment (start 102 123.6625) (end 103.1625 123.6625) (width 0.25) (layer "B.Cu") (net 8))
 (segment (start 103.1625 123.6625) (end 104.2 124.7) (width 0.25) (layer "B.Cu") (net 8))
 (segment (start 91.795001 114.874999) (end 100.574999 114.874999) (width 0.25) (layer "F.Cu") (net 3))
 (segment (start 91.75 114.92) (end 91.795001 114.874999) (width 0.25) (layer "F.Cu") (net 3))
 (segment (start 100.574999 114.874999) (end 101.6 115.9) (width 0.25) (layer "F.Cu") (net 3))
 (via (at 101.6 115.9) (size 0.8) (drill 0.4) (layers "F.Cu" "B.Cu") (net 3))
 (segment (start 105.45 118.05) (end 105.45 120.15) (width 0.25) (layer "B.Cu") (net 3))
 (segment (start 102.2375 117.3) (end 104.7 117.3) (width 0.25) (layer "B.Cu") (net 3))
 (segment (start 105.45 120.15) (end 104.2 121.4) (width 0.25) (layer "B.Cu") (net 3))
 (segment (start 102 117.5375) (end 101.999999 116.299999) (width 0.25) (layer "B.Cu") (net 3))
 (segment (start 102 117.5375) (end 102.2375 117.3) (width 0.25) (layer "B.Cu") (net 3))
 (segment (start 104.7 117.3) (end 105.45 118.05) (width 0.25) (layer "B.Cu") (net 3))
 (segment (start 101.999999 116.299999) (end 101.6 115.9) (width 0.25) (layer "B.Cu") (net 3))
 (segment (start 110.3 123.6) (end 108.8 123.6) (width 0.25) (layer "F.Cu") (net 16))
 (segment (start 113.25 125.08) (end 111.78 125.08) (width 0.25) (layer "F.Cu") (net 16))
 (segment (start 107.7 124.7) (end 106.7 124.7) (width 0.25) (layer "F.Cu") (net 16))
 (segment (start 111.78 125.08) (end 110.3 123.6) (width 0.25) (layer "F.Cu") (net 16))
 (segment (start 108.8 123.6) (end 107.7 124.7) (width 0.25) (layer "F.Cu") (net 16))
 (segment (start 110.6 117.3) (end 110.6 116) (width 0.25) (layer "F.Cu") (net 14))
 (segment (start 111.68 114.92) (end 113.25 114.92) (width 0.25) (layer "F.Cu") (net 14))
 (segment (start 110.6 116) (end 111.68 114.92) (width 0.25) (layer "F.Cu") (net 14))
 (via (at 110.6 117.3) (size 0.8) (drill 0.4) (layers "F.Cu" "B.Cu") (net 14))
 (segment (start 108.55 117.3) (end 110.6 117.3) (width 0.25) (layer "B.Cu") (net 14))
 (segment (start 106.7 121.4) (end 107.95 120.15) (width 0.25) (layer "B.Cu") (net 14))
 (segment (start 107.95 117.9) (end 108.55 117.3) (width 0.25) (layer "B.Cu") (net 14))
 (segment (start 107.95 120.15) (end 107.95 117.9) (width 0.25) (layer "B.Cu") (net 14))
 (segment (start 109.2 124.7) (end 108.4 124.7) (width 0.25) (layer "B.Cu") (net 15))
 (segment (start 102 119.3625) (end 102 121.8375) (width 0.25) (layer "B.Cu") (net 15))
 (segment (start 102.637999 122.475499) (end 107.224501 122.475499) (width 0.25) (layer "B.Cu") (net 15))
 (segment (start 108.6 121.4) (end 109.2 121.4) (width 0.25) (layer "B.Cu") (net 15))
 (segment (start 107.224501 123.524501) (end 107.224501 122.475499) (width 0.25) (layer "B.Cu") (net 15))
 (segment (start 108.4 124.7) (end 107.224501 123.524501) (width 0.25) (layer "B.Cu") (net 15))
 (segment (start 102 121.8375) (end 102.637999 122.475499) (width 0.25) (layer "B.Cu") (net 15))
 (segment (start 107.524501 122.475499) (end 108.6 121.4) (width 0.25) (layer "B.Cu") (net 15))
 (segment (start 107.224501 122.475499) (end 107.524501 122.475499) (width 0.25) (layer "B.Cu") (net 15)))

